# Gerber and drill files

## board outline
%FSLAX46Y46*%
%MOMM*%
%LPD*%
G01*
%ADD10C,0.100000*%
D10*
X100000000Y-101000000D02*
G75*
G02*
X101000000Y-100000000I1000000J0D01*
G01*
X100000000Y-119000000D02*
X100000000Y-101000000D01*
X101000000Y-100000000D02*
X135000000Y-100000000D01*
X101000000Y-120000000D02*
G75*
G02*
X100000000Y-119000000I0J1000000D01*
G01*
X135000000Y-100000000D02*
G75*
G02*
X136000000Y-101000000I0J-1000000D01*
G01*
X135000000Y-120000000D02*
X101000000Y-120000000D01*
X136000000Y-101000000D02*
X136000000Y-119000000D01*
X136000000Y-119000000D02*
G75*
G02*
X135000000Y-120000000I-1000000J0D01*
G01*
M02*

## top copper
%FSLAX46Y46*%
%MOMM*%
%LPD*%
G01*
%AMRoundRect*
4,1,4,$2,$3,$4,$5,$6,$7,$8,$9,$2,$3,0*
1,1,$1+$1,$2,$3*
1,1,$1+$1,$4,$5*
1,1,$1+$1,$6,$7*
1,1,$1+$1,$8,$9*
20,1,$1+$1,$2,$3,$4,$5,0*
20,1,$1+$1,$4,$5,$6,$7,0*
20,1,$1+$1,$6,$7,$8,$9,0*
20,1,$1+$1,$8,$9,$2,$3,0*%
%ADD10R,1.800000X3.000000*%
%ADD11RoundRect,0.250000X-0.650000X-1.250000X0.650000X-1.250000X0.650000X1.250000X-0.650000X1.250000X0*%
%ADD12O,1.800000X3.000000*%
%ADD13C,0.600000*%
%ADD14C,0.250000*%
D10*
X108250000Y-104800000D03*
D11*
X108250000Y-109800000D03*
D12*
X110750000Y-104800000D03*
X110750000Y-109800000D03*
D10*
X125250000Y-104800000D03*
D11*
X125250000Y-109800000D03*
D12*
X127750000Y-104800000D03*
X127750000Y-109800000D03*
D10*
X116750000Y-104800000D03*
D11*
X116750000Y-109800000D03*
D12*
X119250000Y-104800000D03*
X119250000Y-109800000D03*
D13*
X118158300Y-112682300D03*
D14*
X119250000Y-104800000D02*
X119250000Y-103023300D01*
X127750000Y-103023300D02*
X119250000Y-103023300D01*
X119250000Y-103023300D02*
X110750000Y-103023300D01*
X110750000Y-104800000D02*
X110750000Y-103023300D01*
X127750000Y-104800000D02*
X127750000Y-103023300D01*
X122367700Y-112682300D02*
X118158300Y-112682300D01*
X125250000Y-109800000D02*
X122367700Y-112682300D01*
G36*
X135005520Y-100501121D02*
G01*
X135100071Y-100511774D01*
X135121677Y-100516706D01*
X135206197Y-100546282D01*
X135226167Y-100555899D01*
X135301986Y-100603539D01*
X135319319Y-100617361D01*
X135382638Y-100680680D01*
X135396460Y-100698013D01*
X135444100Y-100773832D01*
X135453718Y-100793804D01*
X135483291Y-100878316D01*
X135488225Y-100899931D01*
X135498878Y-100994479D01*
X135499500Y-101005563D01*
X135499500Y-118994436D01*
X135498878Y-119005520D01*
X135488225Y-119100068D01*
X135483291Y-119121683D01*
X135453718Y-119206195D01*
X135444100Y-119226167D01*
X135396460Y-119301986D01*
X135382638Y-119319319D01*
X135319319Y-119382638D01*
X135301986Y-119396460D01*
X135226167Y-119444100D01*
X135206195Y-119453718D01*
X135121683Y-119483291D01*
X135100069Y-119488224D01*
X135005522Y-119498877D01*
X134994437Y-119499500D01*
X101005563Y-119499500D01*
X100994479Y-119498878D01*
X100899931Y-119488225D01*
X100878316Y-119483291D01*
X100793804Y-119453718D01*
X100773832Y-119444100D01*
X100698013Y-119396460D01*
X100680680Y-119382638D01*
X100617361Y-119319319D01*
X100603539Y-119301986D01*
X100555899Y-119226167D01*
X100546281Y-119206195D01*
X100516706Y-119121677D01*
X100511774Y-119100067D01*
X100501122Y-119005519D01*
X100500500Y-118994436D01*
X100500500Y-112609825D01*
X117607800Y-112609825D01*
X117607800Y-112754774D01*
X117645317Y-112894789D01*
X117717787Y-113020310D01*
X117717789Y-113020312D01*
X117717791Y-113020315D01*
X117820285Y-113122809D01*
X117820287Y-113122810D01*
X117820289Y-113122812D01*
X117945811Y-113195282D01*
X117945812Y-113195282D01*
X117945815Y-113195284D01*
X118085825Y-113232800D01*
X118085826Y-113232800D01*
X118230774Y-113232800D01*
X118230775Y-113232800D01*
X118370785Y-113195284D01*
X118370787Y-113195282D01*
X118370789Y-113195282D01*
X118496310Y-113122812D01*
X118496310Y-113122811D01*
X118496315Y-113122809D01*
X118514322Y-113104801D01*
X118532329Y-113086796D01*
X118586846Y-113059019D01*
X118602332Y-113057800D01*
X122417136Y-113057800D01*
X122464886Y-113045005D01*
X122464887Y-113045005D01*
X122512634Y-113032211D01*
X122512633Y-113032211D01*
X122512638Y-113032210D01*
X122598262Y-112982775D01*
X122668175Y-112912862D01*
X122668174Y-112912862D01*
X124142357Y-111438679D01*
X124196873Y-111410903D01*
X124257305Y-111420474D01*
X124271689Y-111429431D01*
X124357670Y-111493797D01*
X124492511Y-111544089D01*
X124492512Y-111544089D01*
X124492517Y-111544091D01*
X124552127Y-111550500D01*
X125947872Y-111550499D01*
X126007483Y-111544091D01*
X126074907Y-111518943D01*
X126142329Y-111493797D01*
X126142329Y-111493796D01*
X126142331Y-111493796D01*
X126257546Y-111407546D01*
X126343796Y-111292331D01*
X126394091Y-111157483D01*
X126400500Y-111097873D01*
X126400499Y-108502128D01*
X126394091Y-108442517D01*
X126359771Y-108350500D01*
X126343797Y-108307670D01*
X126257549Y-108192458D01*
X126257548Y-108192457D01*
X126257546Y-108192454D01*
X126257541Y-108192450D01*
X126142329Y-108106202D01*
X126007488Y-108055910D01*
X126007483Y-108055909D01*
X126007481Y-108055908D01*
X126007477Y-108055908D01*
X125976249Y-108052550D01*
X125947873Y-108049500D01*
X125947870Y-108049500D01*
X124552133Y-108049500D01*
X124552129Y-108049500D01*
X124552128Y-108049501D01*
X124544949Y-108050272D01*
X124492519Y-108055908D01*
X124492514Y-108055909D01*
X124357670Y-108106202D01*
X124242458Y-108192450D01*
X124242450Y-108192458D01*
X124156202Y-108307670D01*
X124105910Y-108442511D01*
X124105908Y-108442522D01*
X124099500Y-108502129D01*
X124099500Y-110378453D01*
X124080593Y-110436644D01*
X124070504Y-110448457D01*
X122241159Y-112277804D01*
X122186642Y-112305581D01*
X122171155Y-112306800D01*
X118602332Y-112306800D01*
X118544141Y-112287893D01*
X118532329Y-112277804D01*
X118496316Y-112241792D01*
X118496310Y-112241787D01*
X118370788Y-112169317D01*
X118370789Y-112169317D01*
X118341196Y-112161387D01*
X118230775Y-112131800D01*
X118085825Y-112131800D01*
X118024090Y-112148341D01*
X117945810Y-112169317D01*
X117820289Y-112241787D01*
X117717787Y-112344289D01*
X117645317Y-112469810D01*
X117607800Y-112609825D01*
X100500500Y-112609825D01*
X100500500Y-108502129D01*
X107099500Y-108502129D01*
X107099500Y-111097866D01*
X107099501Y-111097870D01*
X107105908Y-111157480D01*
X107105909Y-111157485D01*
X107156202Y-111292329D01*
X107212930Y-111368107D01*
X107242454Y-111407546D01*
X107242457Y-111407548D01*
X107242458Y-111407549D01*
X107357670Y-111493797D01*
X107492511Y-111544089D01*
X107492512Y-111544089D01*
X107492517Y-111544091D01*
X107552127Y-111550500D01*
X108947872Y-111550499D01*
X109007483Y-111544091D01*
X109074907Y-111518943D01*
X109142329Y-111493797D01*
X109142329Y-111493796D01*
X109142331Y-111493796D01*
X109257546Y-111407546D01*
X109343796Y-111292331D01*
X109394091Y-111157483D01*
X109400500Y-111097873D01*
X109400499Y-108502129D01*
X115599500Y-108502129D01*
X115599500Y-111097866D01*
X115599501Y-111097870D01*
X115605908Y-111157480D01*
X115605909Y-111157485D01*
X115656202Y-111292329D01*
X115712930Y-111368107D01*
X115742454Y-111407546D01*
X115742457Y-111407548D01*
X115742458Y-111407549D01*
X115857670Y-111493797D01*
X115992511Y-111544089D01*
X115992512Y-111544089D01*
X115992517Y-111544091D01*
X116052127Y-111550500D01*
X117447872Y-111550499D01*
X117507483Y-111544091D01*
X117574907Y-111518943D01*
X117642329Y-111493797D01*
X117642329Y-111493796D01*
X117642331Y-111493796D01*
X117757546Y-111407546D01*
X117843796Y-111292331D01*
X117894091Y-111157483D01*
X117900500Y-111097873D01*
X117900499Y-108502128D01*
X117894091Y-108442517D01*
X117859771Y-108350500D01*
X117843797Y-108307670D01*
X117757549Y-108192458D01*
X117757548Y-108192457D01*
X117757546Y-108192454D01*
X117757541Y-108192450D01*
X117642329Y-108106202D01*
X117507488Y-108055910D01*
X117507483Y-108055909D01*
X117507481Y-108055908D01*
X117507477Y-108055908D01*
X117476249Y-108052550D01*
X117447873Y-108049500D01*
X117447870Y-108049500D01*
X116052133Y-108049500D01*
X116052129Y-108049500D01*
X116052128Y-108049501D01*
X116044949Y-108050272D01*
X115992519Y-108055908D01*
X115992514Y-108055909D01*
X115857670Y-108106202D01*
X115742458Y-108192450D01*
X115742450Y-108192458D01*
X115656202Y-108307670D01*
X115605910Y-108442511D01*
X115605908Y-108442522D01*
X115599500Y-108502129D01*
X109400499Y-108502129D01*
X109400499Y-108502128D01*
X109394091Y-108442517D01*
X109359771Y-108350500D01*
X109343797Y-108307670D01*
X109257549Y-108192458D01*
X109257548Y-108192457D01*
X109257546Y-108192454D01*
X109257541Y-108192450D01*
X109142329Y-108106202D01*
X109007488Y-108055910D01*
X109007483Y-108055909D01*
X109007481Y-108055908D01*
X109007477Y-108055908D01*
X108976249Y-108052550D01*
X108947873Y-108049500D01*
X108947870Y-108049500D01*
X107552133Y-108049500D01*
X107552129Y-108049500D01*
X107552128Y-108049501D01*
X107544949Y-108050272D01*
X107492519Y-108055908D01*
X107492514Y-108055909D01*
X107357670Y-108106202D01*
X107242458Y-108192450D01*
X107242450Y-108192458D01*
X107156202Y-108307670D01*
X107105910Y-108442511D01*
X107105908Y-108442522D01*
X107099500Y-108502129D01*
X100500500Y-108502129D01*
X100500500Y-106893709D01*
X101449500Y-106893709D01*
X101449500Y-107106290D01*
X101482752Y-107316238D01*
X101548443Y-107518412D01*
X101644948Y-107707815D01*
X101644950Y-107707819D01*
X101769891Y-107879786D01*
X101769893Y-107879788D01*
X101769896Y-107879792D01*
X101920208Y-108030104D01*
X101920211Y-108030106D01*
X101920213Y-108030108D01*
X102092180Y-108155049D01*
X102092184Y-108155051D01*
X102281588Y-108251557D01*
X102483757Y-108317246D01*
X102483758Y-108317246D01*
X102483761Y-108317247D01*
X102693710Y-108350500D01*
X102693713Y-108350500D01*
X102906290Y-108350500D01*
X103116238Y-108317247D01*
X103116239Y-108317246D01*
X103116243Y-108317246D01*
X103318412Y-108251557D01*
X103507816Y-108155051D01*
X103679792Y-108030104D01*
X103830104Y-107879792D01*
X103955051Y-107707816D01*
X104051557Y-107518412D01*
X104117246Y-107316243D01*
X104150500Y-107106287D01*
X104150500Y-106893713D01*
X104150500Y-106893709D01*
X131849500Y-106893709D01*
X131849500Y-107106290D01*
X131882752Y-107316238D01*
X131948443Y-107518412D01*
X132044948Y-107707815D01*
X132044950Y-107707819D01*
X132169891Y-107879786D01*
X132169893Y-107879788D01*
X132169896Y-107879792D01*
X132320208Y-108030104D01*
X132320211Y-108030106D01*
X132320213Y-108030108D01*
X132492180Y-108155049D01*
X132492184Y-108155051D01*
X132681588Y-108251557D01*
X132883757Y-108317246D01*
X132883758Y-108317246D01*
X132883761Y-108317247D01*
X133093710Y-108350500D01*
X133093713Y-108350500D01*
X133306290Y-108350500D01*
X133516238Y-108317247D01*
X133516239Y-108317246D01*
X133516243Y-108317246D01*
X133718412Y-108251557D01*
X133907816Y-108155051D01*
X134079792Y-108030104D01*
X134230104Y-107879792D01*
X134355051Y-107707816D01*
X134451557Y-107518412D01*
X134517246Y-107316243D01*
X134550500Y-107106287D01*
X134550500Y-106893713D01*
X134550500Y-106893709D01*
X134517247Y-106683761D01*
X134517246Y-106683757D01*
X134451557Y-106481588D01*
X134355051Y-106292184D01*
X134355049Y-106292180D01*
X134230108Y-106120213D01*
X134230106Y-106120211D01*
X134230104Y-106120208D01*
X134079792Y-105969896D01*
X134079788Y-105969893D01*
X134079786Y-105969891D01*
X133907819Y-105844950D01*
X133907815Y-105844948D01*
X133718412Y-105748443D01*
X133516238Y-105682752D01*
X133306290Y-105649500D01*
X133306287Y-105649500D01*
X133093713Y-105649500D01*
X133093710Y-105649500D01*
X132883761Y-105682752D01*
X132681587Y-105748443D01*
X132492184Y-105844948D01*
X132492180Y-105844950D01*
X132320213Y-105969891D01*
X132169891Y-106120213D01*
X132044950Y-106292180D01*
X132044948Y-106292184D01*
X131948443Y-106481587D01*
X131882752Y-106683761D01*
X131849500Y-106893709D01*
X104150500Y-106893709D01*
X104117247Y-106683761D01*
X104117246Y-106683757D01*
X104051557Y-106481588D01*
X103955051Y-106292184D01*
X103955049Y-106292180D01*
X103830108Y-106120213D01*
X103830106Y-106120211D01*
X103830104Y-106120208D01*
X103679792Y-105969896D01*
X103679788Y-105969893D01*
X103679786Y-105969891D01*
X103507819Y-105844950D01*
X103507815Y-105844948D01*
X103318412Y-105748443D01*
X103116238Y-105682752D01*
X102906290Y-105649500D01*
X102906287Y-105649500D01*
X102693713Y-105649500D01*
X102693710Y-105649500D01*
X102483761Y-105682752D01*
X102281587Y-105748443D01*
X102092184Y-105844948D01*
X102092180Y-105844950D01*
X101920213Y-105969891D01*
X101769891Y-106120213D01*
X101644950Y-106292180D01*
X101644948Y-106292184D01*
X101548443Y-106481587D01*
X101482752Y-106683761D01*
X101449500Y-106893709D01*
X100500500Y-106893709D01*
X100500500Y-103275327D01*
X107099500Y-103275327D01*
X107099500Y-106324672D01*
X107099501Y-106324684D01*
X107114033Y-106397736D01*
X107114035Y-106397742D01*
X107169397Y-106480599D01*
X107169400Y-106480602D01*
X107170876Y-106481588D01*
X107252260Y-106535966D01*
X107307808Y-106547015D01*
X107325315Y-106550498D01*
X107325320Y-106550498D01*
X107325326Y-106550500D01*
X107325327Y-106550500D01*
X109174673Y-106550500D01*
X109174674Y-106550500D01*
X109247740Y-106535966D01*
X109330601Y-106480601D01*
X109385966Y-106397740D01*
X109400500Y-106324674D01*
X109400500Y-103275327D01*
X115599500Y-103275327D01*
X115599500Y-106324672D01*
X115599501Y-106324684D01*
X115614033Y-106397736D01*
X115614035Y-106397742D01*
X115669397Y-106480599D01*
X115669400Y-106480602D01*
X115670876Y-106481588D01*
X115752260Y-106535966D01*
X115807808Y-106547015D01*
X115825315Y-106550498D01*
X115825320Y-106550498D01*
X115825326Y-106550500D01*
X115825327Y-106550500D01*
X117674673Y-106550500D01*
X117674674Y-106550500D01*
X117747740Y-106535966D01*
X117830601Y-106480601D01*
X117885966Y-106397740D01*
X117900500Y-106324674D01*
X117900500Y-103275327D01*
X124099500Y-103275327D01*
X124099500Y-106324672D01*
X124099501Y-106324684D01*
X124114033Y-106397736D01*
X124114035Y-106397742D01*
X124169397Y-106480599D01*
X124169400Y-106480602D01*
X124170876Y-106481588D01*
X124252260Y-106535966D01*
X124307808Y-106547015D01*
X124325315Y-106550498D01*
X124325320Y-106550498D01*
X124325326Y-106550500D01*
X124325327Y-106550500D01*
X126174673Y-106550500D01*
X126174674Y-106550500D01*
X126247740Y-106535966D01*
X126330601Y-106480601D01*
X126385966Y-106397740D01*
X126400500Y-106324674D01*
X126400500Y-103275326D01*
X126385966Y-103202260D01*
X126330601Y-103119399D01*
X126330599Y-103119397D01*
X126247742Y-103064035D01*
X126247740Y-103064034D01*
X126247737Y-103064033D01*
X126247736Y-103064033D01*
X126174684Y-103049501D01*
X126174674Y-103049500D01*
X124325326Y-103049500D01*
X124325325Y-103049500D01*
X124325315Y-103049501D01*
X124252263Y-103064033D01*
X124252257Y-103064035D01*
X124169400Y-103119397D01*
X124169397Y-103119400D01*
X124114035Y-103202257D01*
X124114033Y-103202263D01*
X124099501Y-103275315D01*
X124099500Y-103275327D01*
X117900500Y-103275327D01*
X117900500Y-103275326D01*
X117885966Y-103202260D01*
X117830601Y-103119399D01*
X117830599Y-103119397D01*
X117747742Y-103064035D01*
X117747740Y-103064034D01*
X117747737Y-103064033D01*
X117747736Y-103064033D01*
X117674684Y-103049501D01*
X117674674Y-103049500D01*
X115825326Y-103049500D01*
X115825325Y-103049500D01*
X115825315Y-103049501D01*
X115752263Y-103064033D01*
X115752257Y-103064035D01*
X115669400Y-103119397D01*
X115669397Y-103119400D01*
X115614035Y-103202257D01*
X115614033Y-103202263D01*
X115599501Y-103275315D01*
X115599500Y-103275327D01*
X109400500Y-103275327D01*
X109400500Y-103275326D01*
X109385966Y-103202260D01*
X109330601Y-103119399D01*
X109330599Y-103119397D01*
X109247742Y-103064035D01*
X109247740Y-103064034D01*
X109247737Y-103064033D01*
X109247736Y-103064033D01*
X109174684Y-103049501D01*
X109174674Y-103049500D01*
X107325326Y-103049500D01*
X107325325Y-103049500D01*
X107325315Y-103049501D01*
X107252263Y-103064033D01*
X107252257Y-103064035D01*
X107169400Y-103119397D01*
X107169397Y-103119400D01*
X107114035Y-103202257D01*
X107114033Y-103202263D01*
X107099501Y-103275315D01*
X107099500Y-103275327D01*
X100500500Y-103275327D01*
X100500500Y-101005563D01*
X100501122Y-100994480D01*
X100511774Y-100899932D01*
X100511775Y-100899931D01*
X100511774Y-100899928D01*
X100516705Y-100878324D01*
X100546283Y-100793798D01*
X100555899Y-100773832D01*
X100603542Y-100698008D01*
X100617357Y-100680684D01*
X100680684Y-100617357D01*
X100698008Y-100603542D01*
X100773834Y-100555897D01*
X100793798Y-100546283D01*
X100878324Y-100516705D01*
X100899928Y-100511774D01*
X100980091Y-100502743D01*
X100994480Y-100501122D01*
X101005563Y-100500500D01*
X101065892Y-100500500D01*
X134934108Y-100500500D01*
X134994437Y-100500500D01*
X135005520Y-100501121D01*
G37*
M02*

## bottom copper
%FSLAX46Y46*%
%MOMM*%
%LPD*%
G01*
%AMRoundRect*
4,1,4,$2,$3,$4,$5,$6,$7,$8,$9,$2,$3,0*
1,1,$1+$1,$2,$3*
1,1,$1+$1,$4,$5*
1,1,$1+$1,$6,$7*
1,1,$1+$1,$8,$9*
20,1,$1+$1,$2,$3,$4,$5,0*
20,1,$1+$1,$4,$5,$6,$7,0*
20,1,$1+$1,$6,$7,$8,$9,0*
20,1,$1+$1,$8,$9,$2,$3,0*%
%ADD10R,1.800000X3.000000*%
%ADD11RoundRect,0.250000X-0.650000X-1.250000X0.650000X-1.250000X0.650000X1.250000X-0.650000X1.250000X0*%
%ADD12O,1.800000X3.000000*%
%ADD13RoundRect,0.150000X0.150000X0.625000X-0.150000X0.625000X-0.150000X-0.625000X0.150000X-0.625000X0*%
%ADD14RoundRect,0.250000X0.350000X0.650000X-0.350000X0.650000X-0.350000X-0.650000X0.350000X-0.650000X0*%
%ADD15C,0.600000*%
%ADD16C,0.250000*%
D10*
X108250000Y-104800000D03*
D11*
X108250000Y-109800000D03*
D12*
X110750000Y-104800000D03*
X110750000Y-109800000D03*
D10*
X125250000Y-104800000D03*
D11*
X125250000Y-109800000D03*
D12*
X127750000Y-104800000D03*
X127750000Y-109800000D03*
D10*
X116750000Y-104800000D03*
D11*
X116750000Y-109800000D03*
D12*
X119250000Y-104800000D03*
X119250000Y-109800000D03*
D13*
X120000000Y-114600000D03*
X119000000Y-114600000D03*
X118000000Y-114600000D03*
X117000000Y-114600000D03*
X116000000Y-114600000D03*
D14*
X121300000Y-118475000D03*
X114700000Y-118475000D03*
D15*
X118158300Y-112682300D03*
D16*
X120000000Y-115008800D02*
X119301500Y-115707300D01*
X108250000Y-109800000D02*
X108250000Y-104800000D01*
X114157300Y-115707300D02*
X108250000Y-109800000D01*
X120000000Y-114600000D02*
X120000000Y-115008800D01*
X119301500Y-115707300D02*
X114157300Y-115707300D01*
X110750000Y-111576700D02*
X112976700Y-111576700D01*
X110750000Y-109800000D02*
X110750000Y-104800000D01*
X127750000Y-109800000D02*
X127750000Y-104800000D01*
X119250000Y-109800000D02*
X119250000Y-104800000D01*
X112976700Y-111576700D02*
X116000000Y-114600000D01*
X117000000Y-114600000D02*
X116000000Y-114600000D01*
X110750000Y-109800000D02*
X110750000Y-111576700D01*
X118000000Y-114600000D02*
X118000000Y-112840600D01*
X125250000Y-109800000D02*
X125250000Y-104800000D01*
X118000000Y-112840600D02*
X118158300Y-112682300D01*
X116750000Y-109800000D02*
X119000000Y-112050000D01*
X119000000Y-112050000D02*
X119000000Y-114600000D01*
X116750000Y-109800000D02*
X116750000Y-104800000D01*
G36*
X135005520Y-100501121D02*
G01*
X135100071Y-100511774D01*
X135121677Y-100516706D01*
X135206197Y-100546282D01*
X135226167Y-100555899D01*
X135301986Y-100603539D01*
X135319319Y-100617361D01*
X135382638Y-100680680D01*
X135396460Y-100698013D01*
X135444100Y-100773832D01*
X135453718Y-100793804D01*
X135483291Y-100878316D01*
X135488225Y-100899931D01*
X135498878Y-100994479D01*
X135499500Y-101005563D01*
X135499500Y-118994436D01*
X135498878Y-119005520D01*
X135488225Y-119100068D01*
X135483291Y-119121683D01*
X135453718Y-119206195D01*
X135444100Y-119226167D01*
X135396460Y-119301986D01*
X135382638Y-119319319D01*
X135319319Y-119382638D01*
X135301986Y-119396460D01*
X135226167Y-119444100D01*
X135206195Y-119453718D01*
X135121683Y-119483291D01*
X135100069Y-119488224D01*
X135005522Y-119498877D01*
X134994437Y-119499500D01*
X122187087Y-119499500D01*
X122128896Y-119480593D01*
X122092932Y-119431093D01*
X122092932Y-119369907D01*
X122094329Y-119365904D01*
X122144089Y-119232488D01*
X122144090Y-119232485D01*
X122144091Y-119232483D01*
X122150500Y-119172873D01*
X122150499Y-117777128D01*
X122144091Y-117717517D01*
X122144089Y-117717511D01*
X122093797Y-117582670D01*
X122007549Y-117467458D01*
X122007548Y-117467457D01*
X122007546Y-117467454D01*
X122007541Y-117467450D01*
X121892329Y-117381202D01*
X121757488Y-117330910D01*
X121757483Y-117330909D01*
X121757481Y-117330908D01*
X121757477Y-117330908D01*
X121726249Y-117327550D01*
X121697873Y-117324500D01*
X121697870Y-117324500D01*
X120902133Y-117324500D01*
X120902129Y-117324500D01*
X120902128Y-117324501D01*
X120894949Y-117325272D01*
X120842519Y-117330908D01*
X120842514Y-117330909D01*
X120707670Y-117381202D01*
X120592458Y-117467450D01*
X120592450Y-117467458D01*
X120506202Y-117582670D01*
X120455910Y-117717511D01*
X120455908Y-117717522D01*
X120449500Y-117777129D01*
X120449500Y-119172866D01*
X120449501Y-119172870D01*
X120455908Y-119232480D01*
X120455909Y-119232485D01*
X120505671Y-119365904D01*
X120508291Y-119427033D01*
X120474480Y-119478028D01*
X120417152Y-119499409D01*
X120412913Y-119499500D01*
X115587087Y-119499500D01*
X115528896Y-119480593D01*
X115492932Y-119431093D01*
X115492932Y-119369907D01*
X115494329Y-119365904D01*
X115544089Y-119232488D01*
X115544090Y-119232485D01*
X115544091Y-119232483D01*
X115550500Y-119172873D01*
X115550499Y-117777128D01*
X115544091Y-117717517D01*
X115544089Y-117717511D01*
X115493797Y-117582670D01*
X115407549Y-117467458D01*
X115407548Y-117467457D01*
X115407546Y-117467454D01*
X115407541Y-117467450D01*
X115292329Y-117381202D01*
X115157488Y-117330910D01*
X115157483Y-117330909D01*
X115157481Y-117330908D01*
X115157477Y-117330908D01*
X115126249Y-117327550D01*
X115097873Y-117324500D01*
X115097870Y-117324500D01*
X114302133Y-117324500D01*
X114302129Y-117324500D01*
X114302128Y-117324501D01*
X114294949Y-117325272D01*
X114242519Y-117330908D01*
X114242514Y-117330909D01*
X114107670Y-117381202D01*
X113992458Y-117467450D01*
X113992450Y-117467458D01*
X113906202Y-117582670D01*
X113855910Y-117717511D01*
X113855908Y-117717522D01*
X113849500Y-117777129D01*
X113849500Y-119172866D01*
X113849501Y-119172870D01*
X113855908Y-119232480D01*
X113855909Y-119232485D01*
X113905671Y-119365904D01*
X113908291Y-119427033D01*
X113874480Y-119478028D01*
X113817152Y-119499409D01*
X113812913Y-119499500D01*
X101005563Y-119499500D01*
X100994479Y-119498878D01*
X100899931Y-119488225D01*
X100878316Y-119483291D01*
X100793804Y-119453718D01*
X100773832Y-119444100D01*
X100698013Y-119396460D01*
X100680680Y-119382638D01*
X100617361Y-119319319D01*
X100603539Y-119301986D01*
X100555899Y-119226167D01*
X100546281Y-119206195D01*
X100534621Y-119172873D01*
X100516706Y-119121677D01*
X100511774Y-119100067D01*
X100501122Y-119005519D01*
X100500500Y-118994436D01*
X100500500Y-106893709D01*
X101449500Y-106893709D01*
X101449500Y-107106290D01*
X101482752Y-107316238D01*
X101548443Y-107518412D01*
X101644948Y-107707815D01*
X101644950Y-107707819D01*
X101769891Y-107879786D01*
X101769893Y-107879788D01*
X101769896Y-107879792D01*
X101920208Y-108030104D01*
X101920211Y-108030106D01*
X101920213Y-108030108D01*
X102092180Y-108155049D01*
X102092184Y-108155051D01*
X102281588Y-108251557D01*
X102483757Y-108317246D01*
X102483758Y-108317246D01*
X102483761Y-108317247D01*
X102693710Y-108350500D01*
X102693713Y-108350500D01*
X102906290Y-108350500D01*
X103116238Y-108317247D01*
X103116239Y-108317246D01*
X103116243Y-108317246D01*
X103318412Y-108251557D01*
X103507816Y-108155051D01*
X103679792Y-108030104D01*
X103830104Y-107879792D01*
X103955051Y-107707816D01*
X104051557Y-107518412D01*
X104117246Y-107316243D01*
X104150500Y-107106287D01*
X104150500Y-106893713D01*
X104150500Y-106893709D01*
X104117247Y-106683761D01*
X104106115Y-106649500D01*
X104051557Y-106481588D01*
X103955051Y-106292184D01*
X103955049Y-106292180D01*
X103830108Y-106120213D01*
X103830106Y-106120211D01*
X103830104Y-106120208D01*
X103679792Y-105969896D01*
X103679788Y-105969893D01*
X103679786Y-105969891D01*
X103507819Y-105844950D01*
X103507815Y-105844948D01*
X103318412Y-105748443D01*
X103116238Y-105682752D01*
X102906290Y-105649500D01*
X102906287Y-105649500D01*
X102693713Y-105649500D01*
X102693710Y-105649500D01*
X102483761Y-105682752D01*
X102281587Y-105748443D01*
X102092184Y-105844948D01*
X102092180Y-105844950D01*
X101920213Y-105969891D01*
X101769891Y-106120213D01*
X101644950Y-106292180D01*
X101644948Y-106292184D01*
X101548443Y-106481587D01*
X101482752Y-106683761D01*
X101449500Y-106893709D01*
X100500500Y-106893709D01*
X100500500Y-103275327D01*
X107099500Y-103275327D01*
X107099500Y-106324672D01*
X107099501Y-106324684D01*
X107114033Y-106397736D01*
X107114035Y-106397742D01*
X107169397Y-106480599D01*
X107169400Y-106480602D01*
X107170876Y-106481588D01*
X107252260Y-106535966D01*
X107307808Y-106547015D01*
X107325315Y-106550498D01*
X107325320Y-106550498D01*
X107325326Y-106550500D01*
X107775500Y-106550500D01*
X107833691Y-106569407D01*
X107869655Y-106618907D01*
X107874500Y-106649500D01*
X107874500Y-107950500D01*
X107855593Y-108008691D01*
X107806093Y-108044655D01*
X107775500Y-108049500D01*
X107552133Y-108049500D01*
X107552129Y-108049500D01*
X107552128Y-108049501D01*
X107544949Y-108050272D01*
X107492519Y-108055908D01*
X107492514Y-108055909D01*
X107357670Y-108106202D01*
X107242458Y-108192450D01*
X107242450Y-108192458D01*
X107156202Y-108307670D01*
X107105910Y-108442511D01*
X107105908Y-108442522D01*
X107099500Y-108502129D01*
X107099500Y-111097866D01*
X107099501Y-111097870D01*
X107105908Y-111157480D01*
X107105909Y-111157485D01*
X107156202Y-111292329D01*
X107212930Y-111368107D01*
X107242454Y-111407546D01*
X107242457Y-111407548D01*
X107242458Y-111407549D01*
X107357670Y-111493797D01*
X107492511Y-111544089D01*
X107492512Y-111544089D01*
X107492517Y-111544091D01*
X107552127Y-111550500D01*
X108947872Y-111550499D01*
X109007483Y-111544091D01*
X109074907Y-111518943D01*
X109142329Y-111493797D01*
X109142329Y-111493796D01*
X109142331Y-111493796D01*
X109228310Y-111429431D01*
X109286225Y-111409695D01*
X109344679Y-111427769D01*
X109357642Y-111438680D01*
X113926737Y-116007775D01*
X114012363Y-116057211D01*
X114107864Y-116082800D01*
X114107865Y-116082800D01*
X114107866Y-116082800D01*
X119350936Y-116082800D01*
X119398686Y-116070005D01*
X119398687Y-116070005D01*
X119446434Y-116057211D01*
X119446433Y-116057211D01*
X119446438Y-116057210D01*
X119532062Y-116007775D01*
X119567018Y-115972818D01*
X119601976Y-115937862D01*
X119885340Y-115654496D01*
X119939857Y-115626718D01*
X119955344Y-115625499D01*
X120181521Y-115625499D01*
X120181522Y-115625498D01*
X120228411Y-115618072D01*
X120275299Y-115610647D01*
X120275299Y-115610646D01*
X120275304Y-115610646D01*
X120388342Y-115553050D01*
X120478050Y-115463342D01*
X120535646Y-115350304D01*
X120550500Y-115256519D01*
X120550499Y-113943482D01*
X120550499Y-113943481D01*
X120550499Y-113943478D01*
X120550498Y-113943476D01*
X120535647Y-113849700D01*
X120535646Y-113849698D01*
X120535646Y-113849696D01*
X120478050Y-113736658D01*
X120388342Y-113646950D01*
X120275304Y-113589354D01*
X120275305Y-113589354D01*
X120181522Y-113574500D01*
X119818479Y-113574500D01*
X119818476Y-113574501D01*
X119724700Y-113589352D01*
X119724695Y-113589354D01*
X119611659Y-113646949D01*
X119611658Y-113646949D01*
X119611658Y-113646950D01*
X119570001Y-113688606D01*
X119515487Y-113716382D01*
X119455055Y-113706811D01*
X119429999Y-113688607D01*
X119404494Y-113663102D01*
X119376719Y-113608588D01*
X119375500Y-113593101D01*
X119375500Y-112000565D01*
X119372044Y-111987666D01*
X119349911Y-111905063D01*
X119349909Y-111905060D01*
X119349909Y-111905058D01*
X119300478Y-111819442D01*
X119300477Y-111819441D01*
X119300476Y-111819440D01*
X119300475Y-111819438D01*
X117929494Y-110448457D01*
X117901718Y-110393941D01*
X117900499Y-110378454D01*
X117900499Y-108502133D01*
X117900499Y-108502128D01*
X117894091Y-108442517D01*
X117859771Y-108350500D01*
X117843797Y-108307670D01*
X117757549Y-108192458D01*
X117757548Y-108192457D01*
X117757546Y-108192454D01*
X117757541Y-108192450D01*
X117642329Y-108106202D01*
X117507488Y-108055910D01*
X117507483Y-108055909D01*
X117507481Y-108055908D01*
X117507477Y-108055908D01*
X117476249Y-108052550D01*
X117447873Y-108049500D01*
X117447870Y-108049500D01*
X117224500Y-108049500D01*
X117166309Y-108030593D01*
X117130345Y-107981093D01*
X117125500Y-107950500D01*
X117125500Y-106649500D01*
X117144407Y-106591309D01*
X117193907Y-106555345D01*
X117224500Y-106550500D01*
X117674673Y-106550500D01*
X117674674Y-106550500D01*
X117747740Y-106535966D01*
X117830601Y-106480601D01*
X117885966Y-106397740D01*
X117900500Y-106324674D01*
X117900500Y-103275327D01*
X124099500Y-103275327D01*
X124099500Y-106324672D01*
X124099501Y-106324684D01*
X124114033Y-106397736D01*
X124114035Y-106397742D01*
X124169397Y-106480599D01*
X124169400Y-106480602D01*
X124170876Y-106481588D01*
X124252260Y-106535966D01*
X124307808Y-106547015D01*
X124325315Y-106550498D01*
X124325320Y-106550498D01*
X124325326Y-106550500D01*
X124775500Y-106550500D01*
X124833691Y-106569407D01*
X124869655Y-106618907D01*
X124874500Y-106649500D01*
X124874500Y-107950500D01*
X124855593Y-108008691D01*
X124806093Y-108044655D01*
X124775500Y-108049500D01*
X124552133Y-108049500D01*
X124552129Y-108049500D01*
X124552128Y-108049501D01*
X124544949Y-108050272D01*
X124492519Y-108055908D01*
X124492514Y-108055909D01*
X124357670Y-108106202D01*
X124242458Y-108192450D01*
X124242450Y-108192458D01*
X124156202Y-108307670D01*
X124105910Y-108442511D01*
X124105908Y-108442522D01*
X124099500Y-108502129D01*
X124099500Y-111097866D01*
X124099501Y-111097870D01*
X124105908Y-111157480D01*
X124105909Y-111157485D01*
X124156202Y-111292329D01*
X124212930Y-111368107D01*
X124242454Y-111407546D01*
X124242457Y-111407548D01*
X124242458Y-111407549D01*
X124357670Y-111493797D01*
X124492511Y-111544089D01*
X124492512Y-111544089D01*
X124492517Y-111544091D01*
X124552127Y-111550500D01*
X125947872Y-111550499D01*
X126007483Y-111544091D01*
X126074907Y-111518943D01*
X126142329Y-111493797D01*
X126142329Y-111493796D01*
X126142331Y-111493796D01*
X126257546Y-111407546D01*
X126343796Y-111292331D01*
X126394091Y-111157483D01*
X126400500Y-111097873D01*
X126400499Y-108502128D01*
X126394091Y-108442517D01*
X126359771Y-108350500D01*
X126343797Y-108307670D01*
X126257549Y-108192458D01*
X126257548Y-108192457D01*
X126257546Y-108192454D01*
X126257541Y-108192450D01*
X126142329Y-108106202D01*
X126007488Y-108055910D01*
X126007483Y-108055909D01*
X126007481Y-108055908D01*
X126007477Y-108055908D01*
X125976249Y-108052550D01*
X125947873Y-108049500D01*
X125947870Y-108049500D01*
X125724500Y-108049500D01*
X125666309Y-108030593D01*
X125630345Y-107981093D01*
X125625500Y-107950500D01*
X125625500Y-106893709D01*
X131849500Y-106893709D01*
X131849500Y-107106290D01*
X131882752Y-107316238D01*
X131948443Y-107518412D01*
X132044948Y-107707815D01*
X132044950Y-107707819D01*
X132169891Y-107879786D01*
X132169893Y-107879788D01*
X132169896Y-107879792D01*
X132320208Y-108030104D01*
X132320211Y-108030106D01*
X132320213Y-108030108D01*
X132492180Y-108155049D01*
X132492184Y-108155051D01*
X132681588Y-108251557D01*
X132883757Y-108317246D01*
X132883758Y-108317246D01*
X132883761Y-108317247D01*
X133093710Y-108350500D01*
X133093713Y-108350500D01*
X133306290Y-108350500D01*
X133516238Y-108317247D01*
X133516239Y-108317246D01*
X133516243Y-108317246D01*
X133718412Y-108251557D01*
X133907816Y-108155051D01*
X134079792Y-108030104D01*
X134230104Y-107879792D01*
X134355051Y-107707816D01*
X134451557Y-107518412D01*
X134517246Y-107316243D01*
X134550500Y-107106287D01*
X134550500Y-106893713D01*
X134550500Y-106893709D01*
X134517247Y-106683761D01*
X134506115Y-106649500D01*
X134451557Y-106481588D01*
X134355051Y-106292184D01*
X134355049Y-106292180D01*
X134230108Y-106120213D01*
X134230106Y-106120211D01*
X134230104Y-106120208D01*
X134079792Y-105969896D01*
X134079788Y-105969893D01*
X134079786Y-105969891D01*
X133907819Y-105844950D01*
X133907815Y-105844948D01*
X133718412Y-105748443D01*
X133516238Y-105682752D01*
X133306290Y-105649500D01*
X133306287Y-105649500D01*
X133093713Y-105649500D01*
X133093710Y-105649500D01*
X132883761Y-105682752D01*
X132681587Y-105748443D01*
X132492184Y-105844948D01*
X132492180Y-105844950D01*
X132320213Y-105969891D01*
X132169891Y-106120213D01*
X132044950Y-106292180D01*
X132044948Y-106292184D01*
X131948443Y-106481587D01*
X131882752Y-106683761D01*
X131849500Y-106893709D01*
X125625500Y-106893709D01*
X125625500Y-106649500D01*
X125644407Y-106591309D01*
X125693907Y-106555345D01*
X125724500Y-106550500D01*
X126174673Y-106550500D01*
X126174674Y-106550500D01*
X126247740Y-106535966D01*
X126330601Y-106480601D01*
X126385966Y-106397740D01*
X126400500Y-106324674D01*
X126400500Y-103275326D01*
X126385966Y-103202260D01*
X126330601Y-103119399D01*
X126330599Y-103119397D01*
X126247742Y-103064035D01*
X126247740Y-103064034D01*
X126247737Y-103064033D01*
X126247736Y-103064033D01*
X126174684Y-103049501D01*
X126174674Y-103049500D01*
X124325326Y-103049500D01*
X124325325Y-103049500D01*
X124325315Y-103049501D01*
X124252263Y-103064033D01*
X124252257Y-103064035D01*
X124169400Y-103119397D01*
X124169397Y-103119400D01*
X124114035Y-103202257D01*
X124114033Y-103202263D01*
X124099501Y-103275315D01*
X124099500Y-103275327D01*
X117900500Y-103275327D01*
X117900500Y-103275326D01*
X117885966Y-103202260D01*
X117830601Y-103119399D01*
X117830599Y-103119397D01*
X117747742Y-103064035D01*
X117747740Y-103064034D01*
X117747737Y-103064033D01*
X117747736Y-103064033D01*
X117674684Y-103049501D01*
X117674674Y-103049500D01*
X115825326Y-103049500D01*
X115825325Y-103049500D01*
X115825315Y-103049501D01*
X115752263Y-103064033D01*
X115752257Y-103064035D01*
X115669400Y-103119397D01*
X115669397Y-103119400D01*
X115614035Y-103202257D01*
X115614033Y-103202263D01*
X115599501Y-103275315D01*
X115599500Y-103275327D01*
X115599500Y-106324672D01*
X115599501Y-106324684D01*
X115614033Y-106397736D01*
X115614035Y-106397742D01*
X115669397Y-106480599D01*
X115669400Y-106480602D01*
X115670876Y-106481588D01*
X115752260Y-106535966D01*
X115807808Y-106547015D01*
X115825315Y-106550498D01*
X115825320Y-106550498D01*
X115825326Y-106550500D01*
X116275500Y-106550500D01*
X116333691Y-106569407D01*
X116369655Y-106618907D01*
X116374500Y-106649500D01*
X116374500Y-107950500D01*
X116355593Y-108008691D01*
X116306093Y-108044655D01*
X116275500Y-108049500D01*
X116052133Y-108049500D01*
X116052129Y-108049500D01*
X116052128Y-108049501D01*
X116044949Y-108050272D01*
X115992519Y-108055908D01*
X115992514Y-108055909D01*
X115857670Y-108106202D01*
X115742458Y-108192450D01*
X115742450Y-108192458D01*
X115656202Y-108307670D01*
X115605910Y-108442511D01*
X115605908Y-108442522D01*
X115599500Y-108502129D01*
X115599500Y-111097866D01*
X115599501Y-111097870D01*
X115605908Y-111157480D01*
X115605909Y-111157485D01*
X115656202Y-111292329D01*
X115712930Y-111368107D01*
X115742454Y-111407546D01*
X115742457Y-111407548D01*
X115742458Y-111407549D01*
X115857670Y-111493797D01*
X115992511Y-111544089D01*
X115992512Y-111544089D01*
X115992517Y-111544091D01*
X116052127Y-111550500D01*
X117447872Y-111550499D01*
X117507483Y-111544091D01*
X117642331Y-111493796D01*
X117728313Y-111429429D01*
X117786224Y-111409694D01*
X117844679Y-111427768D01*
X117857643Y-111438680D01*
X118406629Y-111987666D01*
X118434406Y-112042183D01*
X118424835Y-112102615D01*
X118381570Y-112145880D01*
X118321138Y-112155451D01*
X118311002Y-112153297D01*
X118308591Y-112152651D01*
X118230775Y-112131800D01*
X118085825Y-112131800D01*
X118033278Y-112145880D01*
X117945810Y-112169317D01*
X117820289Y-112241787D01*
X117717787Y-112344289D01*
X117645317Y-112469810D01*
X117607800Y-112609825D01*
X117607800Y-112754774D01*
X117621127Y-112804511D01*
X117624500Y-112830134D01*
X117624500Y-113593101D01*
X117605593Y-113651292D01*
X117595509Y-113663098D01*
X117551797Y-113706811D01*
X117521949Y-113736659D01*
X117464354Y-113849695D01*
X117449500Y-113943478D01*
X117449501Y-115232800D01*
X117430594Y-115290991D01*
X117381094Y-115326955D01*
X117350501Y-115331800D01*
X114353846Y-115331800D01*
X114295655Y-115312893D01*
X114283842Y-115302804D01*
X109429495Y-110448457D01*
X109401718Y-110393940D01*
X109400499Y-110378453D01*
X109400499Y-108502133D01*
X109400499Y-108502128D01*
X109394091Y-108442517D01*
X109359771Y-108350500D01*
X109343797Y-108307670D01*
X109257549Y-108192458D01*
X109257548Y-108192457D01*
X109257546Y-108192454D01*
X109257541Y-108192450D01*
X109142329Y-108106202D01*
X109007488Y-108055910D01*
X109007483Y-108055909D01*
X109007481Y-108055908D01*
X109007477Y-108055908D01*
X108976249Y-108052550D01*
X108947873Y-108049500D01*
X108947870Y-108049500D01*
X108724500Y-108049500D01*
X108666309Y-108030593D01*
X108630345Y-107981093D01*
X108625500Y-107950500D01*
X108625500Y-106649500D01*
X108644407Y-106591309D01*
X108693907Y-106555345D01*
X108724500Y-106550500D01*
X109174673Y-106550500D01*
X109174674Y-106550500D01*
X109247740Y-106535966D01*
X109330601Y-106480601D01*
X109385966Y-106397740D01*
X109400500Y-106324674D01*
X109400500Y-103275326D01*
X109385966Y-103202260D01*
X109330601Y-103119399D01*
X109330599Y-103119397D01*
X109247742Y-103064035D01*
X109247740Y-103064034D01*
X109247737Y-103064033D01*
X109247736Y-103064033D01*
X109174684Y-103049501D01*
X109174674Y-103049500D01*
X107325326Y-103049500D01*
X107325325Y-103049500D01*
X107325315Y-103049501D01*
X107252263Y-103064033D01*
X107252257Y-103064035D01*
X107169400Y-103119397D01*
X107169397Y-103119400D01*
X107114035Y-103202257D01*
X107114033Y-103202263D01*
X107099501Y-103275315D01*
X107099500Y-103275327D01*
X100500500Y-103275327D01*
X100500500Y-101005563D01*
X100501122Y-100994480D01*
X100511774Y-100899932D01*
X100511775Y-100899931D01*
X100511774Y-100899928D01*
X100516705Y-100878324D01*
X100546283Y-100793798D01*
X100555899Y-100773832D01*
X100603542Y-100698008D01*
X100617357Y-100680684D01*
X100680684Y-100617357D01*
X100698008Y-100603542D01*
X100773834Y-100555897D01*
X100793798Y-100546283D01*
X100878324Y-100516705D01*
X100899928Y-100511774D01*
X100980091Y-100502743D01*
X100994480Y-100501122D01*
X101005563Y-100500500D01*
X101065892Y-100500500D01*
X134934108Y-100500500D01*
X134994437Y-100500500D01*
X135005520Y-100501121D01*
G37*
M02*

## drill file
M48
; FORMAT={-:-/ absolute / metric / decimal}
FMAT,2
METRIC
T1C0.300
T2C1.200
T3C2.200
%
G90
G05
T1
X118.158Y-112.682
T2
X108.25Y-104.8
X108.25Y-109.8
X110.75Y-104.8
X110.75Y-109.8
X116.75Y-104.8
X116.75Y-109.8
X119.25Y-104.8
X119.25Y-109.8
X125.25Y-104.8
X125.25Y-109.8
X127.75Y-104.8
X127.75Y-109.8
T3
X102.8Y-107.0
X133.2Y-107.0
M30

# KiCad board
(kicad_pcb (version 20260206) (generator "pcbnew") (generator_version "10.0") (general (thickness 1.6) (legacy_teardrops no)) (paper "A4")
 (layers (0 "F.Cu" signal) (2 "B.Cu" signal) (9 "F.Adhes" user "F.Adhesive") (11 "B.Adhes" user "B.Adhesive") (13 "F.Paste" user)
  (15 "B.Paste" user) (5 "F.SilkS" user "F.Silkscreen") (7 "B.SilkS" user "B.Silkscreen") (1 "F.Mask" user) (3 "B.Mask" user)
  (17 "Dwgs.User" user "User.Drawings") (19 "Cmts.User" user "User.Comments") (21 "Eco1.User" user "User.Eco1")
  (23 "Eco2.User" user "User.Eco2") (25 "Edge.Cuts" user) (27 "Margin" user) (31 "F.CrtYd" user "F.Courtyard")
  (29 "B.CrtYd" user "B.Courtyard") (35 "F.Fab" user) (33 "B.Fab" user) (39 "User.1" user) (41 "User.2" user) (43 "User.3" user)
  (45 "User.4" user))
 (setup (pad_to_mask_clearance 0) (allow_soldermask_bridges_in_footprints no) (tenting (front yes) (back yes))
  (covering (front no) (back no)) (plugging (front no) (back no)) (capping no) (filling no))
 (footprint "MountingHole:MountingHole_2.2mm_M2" (layer "F.Cu") (at 102.8 107)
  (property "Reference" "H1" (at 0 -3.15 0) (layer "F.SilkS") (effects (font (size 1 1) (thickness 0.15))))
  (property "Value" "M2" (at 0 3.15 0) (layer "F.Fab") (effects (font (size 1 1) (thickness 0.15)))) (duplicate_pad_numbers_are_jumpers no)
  (pad "" np_thru_hole circle (at 0 0) (size 2.2 2.2) (drill 2.2) (layers "*.Cu" "*.Mask") (zone_connect 2)))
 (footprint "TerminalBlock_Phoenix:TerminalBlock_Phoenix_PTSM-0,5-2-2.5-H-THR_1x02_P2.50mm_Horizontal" (layer "F.Cu") (at 108.25 109.8)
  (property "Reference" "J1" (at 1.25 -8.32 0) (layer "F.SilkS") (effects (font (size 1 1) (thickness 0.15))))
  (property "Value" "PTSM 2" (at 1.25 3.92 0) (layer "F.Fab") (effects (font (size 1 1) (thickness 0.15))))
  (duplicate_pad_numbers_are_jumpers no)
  (pad "1" thru_hole rect (at 0 -5) (size 1.8 3) (drill 1.2) (layers "*.Cu" "*.Mask") (remove_unused_layers no) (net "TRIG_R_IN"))
  (pad "1" thru_hole roundrect (at 0 0) (size 1.8 3) (drill 1.2) (layers "*.Cu" "*.Mask") (remove_unused_layers no)
   (roundrect_rratio 0.138889) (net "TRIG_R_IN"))
  (pad "2" thru_hole oval (at 2.5 -5) (size 1.8 3) (drill 1.2) (layers "*.Cu" "*.Mask") (remove_unused_layers no) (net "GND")
   (zone_connect 2))
  (pad "2" thru_hole oval (at 2.5 0) (size 1.8 3) (drill 1.2) (layers "*.Cu" "*.Mask") (remove_unused_layers no) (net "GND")
   (zone_connect 2)))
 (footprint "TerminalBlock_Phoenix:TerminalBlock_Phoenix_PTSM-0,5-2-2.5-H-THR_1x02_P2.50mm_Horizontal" (layer "F.Cu") (at 125.25 109.8)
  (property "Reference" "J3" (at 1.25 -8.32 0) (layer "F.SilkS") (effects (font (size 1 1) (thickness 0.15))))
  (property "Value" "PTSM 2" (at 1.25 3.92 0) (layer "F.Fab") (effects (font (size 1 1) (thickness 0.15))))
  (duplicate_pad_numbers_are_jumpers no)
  (pad "1" thru_hole rect (at 0 -5) (size 1.8 3) (drill 1.2) (layers "*.Cu" "*.Mask") (remove_unused_layers no) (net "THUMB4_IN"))
  (pad "1" thru_hole roundrect (at 0 0) (size 1.8 3) (drill 1.2) (layers "*.Cu" "*.Mask") (remove_unused_layers no)
   (roundrect_rratio 0.138889) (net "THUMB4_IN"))
  (pad "2" thru_hole oval (at 2.5 -5) (size 1.8 3) (drill 1.2) (layers "*.Cu" "*.Mask") (remove_unused_layers no) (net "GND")
   (zone_connect 2))
  (pad "2" thru_hole oval (at 2.5 0) (size 1.8 3) (drill 1.2) (layers "*.Cu" "*.Mask") (remove_unused_layers no) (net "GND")
   (zone_connect 2)))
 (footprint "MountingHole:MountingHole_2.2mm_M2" (layer "F.Cu") (at 133.2 107)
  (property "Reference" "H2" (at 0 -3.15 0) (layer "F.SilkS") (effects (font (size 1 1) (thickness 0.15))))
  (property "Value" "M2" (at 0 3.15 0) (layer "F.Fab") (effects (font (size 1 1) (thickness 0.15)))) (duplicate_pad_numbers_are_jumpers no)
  (pad "" np_thru_hole circle (at 0 0) (size 2.2 2.2) (drill 2.2) (layers "*.Cu" "*.Mask") (zone_connect 2)))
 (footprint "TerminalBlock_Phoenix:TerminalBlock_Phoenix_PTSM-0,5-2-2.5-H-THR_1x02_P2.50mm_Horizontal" (layer "F.Cu") (at 116.75 109.8)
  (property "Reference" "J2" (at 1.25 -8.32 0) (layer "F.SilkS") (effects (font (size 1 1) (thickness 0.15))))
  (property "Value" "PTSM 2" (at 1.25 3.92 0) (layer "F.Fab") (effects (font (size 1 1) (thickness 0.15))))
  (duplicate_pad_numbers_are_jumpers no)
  (pad "1" thru_hole rect (at 0 -5) (size 1.8 3) (drill 1.2) (layers "*.Cu" "*.Mask") (remove_unused_layers no) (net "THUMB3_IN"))
  (pad "1" thru_hole roundrect (at 0 0) (size 1.8 3) (drill 1.2) (layers "*.Cu" "*.Mask") (remove_unused_layers no)
   (roundrect_rratio 0.138889) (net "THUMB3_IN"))
  (pad "2" thru_hole oval (at 2.5 -5) (size 1.8 3) (drill 1.2) (layers "*.Cu" "*.Mask") (remove_unused_layers no) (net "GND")
   (zone_connect 2))
  (pad "2" thru_hole oval (at 2.5 0) (size 1.8 3) (drill 1.2) (layers "*.Cu" "*.Mask") (remove_unused_layers no) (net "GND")
   (zone_connect 2)))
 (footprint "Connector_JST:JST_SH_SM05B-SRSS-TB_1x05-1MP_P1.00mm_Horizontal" (layer "B.Cu") (at 118 116.6 180)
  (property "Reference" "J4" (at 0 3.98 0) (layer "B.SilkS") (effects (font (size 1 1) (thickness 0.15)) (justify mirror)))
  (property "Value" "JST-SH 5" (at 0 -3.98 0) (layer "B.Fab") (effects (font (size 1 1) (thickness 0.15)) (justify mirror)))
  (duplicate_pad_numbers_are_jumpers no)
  (pad "1" smd roundrect (at -2 2 180) (size 0.6 1.55) (layers "B.Cu" "B.Mask" "B.Paste") (roundrect_rratio 0.25) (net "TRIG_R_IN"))
  (pad "2" smd roundrect (at -1 2 180) (size 0.6 1.55) (layers "B.Cu" "B.Mask" "B.Paste") (roundrect_rratio 0.25) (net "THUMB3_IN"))
  (pad "3" smd roundrect (at 0 2 180) (size 0.6 1.55) (layers "B.Cu" "B.Mask" "B.Paste") (roundrect_rratio 0.25) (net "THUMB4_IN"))
  (pad "4" smd roundrect (at 1 2 180) (size 0.6 1.55) (layers "B.Cu" "B.Mask" "B.Paste") (roundrect_rratio 0.25) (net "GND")
   (zone_connect 2))
  (pad "5" smd roundrect (at 2 2 180) (size 0.6 1.55) (layers "B.Cu" "B.Mask" "B.Paste") (roundrect_rratio 0.25) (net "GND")
   (zone_connect 2))
  (pad "MP" smd roundrect (at -3.3 -1.875 180) (size 1.2 1.8) (layers "B.Cu" "B.Mask" "B.Paste") (roundrect_rratio 0.208333)
   (zone_connect 2))
  (pad "MP" smd roundrect (at 3.3 -1.875 180) (size 1.2 1.8) (layers "B.Cu" "B.Mask" "B.Paste") (roundrect_rratio 0.208333) (zone_connect 2)))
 (gr_arc (start 100 101) (mid 100.292893 100.292893) (end 101 100) (stroke (width 0.1) (type default)) (layer "Edge.Cuts"))
 (gr_line (start 100 119) (end 100 101) (stroke (width 0.1) (type default)) (layer "Edge.Cuts"))
 (gr_line (start 101 100) (end 135 100) (stroke (width 0.1) (type default)) (layer "Edge.Cuts"))
 (gr_arc (start 101 120) (mid 100.292893 119.707107) (end 100 119) (stroke (width 0.1) (type default)) (layer "Edge.Cuts"))
 (gr_arc (start 135 100) (mid 135.707107 100.292893) (end 136 101) (stroke (width 0.1) (type default)) (layer "Edge.Cuts"))
 (gr_line (start 135 120) (end 101 120) (stroke (width 0.1) (type default)) (layer "Edge.Cuts"))
 (gr_line (start 136 101) (end 136 119) (stroke (width 0.1) (type default)) (layer "Edge.Cuts"))
 (gr_arc (start 136 119) (mid 135.707107 119.707107) (end 135 120) (stroke (width 0.1) (type default)) (layer "Edge.Cuts"))
 (segment (start 120 115.0088) (end 119.3015 115.7073) (width 0.25) (layer "B.Cu") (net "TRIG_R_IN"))
 (segment (start 108.25 109.8) (end 108.25 104.8) (width 0.25) (layer "B.Cu") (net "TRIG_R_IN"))
 (segment (start 114.1573 115.7073) (end 108.25 109.8) (width 0.25) (layer "B.Cu") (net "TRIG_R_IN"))
 (segment (start 120 114.6) (end 120 115.0088) (width 0.25) (layer "B.Cu") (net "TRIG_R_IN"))
 (segment (start 119.3015 115.7073) (end 114.1573 115.7073) (width 0.25) (layer "B.Cu") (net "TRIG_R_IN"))
 (segment (start 119.25 104.8) (end 119.25 103.0233) (width 0.25) (layer "F.Cu") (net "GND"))
 (segment (start 127.75 103.0233) (end 119.25 103.0233) (width 0.25) (layer "F.Cu") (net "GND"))
 (segment (start 119.25 103.0233) (end 110.75 103.0233) (width 0.25) (layer "F.Cu") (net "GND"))
 (segment (start 110.75 104.8) (end 110.75 103.0233) (width 0.25) (layer "F.Cu") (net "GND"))
 (segment (start 127.75 104.8) (end 127.75 103.0233) (width 0.25) (layer "F.Cu") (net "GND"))
 (segment (start 110.75 111.5767) (end 112.9767 111.5767) (width 0.25) (layer "B.Cu") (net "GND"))
 (segment (start 110.75 109.8) (end 110.75 104.8) (width 0.25) (layer "B.Cu") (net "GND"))
 (segment (start 127.75 109.8) (end 127.75 104.8) (width 0.25) (layer "B.Cu") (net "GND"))
 (segment (start 119.25 109.8) (end 119.25 104.8) (width 0.25) (layer "B.Cu") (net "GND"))
 (segment (start 112.9767 111.5767) (end 116 114.6) (width 0.25) (layer "B.Cu") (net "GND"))
 (segment (start 117 114.6) (end 116 114.6) (width 0.25) (layer "B.Cu") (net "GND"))
 (segment (start 110.75 109.8) (end 110.75 111.5767) (width 0.25) (layer "B.Cu") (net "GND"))
 (segment (start 122.3677 112.6823) (end 118.1583 112.6823) (width 0.25) (layer "F.Cu") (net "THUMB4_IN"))
 (segment (start 125.25 109.8) (end 122.3677 112.6823) (width 0.25) (layer "F.Cu") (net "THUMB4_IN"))
 (via (at 118.1583 112.6823) (size 0.6) (drill 0.3) (layers "F.Cu" "B.Cu") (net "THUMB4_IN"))
 (segment (start 118 114.6) (end 118 112.8406) (width 0.25) (layer "B.Cu") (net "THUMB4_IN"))
 (segment (start 125.25 109.8) (end 125.25 104.8) (width 0.25) (layer "B.Cu") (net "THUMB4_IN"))
 (segment (start 118 112.8406) (end 118.1583 112.6823) (width 0.25) (layer "B.Cu") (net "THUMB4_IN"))
 (segment (start 116.75 109.8) (end 119 112.05) (width 0.25) (layer "B.Cu") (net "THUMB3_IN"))
 (segment (start 119 112.05) (end 119 114.6) (width 0.25) (layer "B.Cu") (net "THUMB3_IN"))
 (segment (start 116.75 109.8) (end 116.75 104.8) (width 0.25) (layer "B.Cu") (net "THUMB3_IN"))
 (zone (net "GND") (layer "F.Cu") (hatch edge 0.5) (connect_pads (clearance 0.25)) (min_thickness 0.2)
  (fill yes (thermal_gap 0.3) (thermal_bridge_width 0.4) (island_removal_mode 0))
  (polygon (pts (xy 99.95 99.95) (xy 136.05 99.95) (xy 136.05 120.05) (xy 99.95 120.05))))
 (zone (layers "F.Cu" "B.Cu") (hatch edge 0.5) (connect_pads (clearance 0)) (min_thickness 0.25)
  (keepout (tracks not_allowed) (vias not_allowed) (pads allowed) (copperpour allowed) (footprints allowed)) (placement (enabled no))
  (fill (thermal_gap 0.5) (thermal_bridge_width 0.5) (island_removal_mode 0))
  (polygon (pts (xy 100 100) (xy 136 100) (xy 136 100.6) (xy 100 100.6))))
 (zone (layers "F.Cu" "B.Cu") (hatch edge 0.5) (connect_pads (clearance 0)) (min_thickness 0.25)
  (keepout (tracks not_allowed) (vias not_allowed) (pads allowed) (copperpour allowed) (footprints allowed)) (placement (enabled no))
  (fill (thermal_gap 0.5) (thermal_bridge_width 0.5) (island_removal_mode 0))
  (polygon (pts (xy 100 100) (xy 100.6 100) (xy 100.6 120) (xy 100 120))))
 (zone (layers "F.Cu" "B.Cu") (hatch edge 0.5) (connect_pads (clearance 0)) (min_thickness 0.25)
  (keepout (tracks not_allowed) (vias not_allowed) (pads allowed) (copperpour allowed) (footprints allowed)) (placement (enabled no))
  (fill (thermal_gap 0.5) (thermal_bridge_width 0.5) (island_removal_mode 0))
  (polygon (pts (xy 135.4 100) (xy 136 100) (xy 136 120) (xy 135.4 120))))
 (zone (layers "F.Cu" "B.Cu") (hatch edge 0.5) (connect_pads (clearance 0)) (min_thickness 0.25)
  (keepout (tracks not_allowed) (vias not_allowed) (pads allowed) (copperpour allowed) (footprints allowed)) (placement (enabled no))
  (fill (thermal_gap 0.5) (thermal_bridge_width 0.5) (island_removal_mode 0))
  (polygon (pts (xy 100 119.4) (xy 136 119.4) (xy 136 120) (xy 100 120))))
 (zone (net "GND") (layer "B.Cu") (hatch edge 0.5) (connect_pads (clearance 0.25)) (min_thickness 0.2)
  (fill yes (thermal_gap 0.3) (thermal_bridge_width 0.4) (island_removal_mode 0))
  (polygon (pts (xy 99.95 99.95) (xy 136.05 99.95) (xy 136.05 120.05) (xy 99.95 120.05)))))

